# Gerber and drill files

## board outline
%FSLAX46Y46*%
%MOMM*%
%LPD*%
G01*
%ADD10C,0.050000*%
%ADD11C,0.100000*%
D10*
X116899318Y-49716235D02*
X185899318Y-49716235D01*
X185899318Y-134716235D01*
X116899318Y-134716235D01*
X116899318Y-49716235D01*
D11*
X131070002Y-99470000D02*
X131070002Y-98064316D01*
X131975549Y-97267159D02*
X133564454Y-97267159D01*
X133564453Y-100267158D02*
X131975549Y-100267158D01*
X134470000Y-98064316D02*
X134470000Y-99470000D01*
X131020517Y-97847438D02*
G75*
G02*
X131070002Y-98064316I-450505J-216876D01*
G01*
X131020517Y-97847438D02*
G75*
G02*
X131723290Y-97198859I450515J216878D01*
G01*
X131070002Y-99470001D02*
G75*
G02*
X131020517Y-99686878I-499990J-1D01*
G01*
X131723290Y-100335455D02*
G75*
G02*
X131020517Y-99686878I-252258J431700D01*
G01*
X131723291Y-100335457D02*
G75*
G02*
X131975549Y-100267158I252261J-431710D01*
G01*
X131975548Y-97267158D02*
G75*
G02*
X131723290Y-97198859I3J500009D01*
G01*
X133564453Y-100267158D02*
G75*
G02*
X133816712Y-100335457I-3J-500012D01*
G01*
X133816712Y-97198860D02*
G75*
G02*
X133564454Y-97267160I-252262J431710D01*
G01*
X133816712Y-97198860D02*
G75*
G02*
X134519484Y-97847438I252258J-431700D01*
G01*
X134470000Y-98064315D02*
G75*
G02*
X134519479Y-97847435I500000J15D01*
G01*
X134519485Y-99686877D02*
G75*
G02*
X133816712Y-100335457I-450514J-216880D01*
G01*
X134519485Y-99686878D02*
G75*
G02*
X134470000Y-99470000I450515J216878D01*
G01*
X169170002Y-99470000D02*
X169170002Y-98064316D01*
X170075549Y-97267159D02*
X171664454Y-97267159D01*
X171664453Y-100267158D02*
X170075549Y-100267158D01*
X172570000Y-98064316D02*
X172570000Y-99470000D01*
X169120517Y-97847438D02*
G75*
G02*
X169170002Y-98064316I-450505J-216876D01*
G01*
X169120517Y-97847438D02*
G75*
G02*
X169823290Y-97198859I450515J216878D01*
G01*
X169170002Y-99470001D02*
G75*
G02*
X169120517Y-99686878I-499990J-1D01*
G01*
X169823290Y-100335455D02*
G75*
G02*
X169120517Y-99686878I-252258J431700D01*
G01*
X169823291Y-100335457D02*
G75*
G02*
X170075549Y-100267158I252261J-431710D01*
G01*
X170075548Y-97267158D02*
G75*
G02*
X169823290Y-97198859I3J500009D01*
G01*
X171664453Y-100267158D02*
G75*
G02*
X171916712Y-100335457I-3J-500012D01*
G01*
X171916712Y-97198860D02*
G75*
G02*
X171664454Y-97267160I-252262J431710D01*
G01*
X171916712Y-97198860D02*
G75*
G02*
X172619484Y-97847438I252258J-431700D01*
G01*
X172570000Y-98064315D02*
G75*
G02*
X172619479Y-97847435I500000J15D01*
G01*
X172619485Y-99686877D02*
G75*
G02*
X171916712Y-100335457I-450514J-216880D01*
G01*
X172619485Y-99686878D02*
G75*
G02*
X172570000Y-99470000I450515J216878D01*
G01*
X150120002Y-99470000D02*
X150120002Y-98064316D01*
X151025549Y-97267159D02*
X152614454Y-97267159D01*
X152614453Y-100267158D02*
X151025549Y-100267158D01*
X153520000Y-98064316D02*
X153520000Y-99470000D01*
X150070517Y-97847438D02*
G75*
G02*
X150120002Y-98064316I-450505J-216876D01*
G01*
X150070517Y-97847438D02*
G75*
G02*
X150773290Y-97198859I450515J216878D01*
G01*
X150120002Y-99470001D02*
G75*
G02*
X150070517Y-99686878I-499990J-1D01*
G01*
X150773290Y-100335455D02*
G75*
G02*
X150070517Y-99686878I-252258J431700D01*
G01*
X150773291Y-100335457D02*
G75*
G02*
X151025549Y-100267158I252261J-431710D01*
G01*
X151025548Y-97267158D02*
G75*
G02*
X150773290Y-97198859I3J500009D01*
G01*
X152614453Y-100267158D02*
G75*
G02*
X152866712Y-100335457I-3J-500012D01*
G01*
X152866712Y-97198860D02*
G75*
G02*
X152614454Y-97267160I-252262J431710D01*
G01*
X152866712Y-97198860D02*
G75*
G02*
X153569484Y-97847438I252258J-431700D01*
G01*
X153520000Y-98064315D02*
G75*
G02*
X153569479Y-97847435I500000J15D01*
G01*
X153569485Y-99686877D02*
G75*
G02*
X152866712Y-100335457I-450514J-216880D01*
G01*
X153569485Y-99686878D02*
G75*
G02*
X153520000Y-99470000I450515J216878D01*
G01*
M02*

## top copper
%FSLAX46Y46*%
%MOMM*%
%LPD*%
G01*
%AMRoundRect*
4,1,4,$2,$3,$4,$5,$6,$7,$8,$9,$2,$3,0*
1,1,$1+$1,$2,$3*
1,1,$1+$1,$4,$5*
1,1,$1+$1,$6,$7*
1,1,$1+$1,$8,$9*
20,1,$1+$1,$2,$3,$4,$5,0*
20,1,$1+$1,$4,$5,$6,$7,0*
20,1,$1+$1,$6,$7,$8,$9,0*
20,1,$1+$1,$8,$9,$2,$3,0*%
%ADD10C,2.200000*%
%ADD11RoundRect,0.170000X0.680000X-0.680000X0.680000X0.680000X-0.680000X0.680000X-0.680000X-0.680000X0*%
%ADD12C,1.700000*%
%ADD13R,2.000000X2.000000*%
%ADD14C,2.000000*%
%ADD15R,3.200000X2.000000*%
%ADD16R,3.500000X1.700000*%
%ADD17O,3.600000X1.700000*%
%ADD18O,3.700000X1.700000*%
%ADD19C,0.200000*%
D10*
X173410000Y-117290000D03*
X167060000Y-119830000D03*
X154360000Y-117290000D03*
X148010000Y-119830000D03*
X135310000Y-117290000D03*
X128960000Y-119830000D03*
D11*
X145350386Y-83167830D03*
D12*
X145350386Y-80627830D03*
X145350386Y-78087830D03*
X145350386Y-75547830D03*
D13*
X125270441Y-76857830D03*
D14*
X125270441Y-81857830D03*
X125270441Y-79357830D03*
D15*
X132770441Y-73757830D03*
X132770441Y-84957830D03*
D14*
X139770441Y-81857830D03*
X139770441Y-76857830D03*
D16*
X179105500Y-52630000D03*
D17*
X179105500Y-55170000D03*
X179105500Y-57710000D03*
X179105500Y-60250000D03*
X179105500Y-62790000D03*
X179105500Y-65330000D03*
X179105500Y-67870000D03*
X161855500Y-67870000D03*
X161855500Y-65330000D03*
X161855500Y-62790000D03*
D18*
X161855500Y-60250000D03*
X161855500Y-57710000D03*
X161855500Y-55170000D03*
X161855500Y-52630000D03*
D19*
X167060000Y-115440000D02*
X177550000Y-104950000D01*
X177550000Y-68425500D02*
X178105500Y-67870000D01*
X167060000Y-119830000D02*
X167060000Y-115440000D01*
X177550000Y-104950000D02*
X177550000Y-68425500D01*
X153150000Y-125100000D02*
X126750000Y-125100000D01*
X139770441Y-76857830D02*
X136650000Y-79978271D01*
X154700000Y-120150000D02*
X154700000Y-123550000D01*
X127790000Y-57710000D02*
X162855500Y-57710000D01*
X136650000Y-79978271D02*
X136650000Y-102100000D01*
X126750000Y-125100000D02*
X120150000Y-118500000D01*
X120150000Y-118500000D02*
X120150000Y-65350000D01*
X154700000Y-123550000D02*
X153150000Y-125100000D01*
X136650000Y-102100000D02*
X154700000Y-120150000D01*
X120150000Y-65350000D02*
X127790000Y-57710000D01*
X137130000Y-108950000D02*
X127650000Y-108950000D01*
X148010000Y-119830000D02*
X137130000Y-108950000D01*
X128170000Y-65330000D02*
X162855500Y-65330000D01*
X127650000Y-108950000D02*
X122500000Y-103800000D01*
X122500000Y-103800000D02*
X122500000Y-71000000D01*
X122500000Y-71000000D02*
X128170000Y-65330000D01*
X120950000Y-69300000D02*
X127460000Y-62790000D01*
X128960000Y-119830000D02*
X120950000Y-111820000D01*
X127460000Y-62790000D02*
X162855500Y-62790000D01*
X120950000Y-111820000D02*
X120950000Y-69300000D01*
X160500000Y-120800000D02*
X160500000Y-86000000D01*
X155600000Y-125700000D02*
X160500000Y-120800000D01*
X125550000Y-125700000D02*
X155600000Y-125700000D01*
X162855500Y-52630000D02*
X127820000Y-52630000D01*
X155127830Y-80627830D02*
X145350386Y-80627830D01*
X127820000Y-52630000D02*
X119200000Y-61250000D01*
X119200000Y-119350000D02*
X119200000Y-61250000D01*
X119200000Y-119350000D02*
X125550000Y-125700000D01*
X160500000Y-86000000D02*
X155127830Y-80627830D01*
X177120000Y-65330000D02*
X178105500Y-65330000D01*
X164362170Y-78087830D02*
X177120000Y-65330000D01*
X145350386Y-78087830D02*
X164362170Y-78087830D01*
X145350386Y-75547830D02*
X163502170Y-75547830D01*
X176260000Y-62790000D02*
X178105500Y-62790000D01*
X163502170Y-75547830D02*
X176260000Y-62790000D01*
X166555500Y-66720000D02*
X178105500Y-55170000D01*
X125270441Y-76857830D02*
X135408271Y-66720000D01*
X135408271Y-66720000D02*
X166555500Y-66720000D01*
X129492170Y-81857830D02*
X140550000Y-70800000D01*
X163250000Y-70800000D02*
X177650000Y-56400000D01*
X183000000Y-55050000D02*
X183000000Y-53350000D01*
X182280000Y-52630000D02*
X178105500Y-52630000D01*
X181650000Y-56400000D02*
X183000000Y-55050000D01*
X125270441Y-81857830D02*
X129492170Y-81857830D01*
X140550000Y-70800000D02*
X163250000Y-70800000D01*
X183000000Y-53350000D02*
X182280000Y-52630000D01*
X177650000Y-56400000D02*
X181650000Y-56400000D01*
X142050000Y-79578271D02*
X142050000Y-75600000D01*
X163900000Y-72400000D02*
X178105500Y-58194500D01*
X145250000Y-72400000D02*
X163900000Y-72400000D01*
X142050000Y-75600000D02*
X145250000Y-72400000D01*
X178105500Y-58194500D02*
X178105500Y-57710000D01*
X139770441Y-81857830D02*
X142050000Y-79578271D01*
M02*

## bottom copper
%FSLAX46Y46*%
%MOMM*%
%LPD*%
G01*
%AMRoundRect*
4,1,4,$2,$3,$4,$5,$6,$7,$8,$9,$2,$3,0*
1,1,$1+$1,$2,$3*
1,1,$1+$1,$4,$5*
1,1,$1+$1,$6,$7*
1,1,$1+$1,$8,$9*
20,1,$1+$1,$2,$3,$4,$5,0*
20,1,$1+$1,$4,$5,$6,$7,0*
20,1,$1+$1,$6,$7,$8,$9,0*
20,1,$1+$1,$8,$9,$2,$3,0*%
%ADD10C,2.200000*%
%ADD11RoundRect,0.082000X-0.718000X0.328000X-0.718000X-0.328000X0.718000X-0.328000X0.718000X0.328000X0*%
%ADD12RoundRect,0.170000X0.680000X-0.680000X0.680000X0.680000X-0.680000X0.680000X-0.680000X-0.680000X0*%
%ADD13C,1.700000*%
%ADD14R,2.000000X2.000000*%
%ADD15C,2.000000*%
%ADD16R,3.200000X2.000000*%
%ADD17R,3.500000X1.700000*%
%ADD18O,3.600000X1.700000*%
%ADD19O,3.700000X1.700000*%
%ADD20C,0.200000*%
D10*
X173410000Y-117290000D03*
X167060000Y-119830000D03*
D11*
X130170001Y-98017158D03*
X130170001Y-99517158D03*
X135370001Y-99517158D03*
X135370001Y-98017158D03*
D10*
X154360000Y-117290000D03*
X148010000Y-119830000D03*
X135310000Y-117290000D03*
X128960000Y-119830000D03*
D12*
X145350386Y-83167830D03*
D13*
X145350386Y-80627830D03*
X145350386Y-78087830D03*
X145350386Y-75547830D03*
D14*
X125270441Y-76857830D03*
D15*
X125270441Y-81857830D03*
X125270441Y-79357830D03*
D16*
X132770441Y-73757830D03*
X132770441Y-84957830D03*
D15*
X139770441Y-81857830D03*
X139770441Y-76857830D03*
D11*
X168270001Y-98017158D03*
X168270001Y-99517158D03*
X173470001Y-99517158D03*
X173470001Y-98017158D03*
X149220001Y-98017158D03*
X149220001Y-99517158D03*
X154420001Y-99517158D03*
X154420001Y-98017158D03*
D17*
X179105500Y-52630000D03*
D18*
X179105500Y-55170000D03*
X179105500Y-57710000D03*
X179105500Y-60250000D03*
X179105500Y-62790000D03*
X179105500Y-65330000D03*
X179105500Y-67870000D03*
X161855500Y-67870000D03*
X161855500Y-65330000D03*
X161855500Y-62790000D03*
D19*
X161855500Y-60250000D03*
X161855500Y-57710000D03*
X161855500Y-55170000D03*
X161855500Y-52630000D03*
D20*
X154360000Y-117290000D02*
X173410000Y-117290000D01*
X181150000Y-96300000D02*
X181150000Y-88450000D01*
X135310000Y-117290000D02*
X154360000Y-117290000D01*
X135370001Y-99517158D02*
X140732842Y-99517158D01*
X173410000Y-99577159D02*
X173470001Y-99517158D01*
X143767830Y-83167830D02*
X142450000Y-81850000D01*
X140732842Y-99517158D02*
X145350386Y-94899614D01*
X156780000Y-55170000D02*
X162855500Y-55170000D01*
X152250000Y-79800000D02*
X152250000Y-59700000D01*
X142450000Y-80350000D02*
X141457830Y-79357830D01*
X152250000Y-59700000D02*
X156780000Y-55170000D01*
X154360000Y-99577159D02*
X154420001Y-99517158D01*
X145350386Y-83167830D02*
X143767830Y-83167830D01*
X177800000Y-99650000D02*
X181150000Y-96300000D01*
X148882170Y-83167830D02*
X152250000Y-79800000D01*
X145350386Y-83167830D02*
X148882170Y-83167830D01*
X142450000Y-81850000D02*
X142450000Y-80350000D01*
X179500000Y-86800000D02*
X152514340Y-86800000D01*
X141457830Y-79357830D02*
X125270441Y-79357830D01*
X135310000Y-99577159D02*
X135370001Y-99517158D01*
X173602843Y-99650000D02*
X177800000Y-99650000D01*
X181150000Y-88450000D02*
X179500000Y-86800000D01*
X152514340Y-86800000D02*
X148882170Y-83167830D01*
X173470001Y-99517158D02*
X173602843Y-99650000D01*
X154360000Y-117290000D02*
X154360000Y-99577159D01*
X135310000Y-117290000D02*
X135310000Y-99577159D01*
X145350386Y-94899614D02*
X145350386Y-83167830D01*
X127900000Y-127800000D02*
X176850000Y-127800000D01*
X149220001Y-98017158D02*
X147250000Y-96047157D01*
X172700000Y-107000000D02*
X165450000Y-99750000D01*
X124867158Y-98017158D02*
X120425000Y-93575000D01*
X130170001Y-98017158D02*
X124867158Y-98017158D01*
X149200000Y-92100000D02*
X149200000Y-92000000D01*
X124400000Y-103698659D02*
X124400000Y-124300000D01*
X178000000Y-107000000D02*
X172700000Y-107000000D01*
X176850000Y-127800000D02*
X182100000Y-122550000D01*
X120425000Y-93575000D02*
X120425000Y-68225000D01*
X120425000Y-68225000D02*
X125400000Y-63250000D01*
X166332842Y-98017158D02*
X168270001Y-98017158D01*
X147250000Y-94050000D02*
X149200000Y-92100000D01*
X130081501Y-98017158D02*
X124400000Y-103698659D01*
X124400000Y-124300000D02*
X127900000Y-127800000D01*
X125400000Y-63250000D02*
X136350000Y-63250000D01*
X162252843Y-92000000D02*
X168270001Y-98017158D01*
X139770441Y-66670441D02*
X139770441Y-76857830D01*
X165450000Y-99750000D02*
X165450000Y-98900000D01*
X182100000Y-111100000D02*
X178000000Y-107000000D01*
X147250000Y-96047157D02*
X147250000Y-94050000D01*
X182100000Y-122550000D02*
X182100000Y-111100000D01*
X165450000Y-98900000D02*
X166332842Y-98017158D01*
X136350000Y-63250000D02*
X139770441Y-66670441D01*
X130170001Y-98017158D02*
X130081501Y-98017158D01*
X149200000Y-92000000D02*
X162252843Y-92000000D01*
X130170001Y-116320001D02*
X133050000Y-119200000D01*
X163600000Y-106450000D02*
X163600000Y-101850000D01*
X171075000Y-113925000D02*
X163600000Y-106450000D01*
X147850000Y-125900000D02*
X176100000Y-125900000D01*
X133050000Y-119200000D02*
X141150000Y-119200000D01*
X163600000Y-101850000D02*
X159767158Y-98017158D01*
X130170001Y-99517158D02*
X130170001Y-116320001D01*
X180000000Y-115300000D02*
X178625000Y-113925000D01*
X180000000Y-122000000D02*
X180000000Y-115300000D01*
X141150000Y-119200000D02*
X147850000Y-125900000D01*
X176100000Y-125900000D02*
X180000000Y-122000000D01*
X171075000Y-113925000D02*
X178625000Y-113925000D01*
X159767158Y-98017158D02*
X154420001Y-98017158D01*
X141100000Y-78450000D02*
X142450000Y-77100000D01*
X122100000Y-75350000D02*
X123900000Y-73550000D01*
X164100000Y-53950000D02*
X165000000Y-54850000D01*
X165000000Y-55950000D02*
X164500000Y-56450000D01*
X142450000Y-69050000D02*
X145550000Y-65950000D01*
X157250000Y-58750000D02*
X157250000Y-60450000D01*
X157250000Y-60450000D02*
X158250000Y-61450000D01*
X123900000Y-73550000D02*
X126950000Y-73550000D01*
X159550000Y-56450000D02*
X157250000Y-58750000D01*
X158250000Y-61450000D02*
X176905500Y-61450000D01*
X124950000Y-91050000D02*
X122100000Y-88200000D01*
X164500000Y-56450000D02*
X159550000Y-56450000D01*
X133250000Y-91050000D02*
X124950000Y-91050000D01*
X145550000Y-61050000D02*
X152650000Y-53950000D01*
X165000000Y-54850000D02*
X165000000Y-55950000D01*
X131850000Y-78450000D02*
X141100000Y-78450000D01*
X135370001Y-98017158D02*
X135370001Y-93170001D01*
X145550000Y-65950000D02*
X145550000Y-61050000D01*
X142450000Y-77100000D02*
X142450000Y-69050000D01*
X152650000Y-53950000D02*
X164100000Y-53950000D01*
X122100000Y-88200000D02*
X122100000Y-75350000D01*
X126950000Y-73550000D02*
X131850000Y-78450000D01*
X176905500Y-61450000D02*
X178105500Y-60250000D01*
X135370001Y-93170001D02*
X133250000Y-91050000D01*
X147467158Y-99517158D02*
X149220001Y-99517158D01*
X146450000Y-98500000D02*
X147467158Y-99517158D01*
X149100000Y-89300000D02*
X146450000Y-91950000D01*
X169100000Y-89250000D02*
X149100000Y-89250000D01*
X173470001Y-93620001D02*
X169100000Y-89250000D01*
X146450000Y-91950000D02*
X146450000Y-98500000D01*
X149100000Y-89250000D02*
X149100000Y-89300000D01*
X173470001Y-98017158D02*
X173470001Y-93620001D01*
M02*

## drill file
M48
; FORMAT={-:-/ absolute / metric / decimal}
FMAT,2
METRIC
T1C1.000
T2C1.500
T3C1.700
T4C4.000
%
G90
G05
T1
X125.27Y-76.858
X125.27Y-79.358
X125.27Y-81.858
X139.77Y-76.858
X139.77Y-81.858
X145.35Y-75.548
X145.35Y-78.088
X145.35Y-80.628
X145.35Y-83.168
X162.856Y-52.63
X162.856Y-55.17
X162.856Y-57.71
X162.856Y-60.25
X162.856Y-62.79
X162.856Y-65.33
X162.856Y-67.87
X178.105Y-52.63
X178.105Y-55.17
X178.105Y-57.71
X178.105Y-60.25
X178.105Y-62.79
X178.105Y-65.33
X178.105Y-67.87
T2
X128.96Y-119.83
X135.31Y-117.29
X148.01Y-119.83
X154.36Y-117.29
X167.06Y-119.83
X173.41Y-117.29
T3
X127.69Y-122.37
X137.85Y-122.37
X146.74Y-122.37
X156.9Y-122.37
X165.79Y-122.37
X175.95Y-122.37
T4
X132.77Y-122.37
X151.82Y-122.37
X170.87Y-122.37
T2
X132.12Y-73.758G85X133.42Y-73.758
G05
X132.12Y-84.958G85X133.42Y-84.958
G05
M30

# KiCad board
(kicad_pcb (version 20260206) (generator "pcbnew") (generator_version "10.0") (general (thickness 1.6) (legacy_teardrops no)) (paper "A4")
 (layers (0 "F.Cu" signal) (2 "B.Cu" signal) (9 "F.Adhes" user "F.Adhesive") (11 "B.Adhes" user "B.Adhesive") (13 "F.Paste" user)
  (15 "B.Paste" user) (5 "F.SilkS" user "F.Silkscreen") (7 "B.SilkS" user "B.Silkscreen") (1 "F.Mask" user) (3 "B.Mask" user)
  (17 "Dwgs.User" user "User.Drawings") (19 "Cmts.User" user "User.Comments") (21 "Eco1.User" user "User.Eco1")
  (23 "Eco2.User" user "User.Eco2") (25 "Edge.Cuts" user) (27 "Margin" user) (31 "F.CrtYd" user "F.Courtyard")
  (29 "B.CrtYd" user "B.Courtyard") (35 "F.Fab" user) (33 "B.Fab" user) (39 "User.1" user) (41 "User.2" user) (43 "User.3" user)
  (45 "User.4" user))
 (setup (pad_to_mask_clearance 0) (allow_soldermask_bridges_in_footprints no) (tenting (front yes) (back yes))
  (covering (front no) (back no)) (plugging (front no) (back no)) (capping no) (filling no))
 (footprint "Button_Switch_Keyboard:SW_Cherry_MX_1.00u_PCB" (layer "F.Cu") (at 173.41 117.29)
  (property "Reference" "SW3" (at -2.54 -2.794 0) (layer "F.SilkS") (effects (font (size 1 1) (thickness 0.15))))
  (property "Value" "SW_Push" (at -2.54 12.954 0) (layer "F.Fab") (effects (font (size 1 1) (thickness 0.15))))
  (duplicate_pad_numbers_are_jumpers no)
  (pad "" np_thru_hole circle (at -7.62 5.08) (size 1.7 1.7) (drill 1.7) (layers "*.Cu" "*.Mask"))
  (pad "" np_thru_hole circle (at -2.54 5.08) (size 4 4) (drill 4) (layers "*.Cu" "*.Mask"))
  (pad "" np_thru_hole circle (at 2.54 5.08) (size 1.7 1.7) (drill 1.7) (layers "*.Cu" "*.Mask"))
  (pad "1" thru_hole circle (at 0 0) (size 2.2 2.2) (drill 1.5) (layers "*.Cu" "*.Mask") (remove_unused_layers no) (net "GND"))
  (pad "2" thru_hole circle (at -6.35 2.54) (size 2.2 2.2) (drill 1.5) (layers "*.Cu" "*.Mask") (remove_unused_layers no)
   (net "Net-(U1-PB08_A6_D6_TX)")))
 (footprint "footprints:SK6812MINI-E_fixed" (layer "F.Cu") (at 132.77 98.87)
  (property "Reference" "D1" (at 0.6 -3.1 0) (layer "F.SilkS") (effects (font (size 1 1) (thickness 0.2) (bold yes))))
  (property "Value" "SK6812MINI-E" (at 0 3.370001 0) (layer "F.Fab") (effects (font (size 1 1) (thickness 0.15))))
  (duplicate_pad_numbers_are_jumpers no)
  (fp_line (start -1.699998 0.6) (end -1.699998 -0.805684) (stroke (width 0.1) (type solid)) (layer "Edge.Cuts"))
  (fp_line (start -0.794451 -1.602841) (end 0.794454 -1.602841) (stroke (width 0.1) (type solid)) (layer "Edge.Cuts"))
  (fp_line (start 0.794453 1.397158) (end -0.794451 1.397158) (stroke (width 0.1) (type solid)) (layer "Edge.Cuts"))
  (fp_line (start 1.7 -0.805684) (end 1.7 0.6) (stroke (width 0.1) (type solid)) (layer "Edge.Cuts"))
  (fp_arc (start -1.749483 -1.022562) (mid -1.712526 -0.91691) (end -1.699998 -0.805684) (stroke (width 0.1) (type solid))
   (layer "Edge.Cuts"))
  (fp_arc (start -1.749483 -1.022562) (mid -1.63807 -1.606877) (end -1.04671 -1.671141) (stroke (width 0.1) (type solid))
   (layer "Edge.Cuts"))
  (fp_arc (start -1.699998 0.600001) (mid -1.712526 0.711226) (end -1.749483 0.816878) (stroke (width 0.1) (type solid)) (layer "Edge.Cuts"))
  (fp_arc (start -1.04671 1.465455) (mid -1.638069 1.401192) (end -1.749483 0.816878) (stroke (width 0.1) (type solid)) (layer "Edge.Cuts"))
  (fp_arc (start -1.046709 1.465457) (mid -0.925121 1.414535) (end -0.794451 1.397158) (stroke (width 0.1) (type solid)) (layer "Edge.Cuts"))
  (fp_arc (start -0.794452 -1.602842) (mid -0.925122 -1.620219) (end -1.04671 -1.671141) (stroke (width 0.1) (type solid))
   (layer "Edge.Cuts"))
  (fp_arc (start 0.794453 1.397158) (mid 0.925124 1.414535) (end 1.046712 1.465457) (stroke (width 0.1) (type solid)) (layer "Edge.Cuts"))
  (fp_arc (start 1.046712 -1.67114) (mid 0.925124 -1.620218) (end 0.794454 -1.602841) (stroke (width 0.1) (type solid)) (layer "Edge.Cuts"))
  (fp_arc (start 1.046712 -1.67114) (mid 1.638072 -1.606876) (end 1.749485 -1.022562) (stroke (width 0.1) (type solid)) (layer "Edge.Cuts"))
  (fp_arc (start 1.7 -0.805685) (mid 1.712528 -0.91691) (end 1.749485 -1.022562) (stroke (width 0.1) (type solid)) (layer "Edge.Cuts"))
  (fp_arc (start 1.749485 0.816877) (mid 1.638073 1.401193) (end 1.046712 1.465457) (stroke (width 0.1) (type solid)) (layer "Edge.Cuts"))
  (fp_arc (start 1.749485 0.816878) (mid 1.712528 0.711226) (end 1.7 0.6) (stroke (width 0.1) (type solid)) (layer "Edge.Cuts"))
  (pad "1" smd roundrect (at -2.599999 -0.852842 270) (size 0.82 1.6) (layers "B.Cu" "B.Mask" "B.Paste") (roundrect_rratio 0.1)
   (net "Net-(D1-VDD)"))
  (pad "2" smd roundrect (at -2.599999 0.647158 270) (size 0.82 1.6) (layers "B.Cu" "B.Mask" "B.Paste") (roundrect_rratio 0.1)
   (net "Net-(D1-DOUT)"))
  (pad "3" smd roundrect (at 2.600001 0.647158 270) (size 0.82 1.6) (layers "B.Cu" "B.Mask" "B.Paste") (roundrect_rratio 0.1) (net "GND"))
  (pad "4" smd roundrect (at 2.600001 -0.852842 270) (size 0.82 1.6) (layers "B.Cu" "B.Mask" "B.Paste") (roundrect_rratio 0.1)
   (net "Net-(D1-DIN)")))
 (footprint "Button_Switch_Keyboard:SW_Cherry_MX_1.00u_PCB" (layer "F.Cu") (at 154.36 117.29)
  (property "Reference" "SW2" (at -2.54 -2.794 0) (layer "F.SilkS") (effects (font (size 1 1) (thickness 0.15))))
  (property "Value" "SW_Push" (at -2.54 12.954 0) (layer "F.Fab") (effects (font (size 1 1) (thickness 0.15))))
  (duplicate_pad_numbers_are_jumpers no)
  (pad "" np_thru_hole circle (at -7.62 5.08) (size 1.7 1.7) (drill 1.7) (layers "*.Cu" "*.Mask"))
  (pad "" np_thru_hole circle (at -2.54 5.08) (size 4 4) (drill 4) (layers "*.Cu" "*.Mask"))
  (pad "" np_thru_hole circle (at 2.54 5.08) (size 1.7 1.7) (drill 1.7) (layers "*.Cu" "*.Mask"))
  (pad "1" thru_hole circle (at 0 0) (size 2.2 2.2) (drill 1.5) (layers "*.Cu" "*.Mask") (remove_unused_layers no) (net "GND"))
  (pad "2" thru_hole circle (at -6.35 2.54) (size 2.2 2.2) (drill 1.5) (layers "*.Cu" "*.Mask") (remove_unused_layers no)
   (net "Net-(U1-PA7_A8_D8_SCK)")))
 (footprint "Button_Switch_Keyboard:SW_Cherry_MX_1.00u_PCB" (layer "F.Cu") (at 135.31 117.29)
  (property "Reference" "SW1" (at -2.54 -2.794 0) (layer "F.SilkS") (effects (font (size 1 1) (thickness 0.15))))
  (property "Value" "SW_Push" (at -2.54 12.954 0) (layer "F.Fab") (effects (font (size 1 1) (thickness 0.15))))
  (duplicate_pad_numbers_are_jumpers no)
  (pad "" np_thru_hole circle (at -7.62 5.08) (size 1.7 1.7) (drill 1.7) (layers "*.Cu" "*.Mask"))
  (pad "" np_thru_hole circle (at -2.54 5.08) (size 4 4) (drill 4) (layers "*.Cu" "*.Mask"))
  (pad "" np_thru_hole circle (at 2.54 5.08) (size 1.7 1.7) (drill 1.7) (layers "*.Cu" "*.Mask"))
  (pad "1" thru_hole circle (at 0 0) (size 2.2 2.2) (drill 1.5) (layers "*.Cu" "*.Mask") (remove_unused_layers no) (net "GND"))
  (pad "2" thru_hole circle (at -6.35 2.54) (size 2.2 2.2) (drill 1.5) (layers "*.Cu" "*.Mask") (remove_unused_layers no)
   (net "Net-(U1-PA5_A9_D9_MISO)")))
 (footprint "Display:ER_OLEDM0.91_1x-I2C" (layer "F.Cu") (at 145.350386 83.16783 90)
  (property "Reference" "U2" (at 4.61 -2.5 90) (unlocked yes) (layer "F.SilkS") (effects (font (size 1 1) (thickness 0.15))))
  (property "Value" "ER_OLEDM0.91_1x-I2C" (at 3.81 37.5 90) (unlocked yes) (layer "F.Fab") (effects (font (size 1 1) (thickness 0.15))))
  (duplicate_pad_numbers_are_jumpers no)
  (pad "1" thru_hole roundrect (at 0 0 90) (size 1.7 1.7) (drill 1) (layers "*.Cu" "*.Mask") (remove_unused_layers no)
   (roundrect_rratio 0.1) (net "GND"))
  (pad "2" thru_hole circle (at 2.54 0 90) (size 1.7 1.7) (drill 1) (layers "*.Cu" "*.Mask") (remove_unused_layers no) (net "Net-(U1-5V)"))
  (pad "3" thru_hole circle (at 5.08 0 90) (size 1.7 1.7) (drill 1) (layers "*.Cu" "*.Mask") (remove_unused_layers no)
   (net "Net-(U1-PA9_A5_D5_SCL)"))
  (pad "4" thru_hole circle (at 7.62 0 90) (size 1.7 1.7) (drill 1) (layers "*.Cu" "*.Mask") (remove_unused_layers no)
   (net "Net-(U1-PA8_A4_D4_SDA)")))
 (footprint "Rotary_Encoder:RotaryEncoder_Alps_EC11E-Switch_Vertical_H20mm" (layer "F.Cu") (at 125.270441 76.85783)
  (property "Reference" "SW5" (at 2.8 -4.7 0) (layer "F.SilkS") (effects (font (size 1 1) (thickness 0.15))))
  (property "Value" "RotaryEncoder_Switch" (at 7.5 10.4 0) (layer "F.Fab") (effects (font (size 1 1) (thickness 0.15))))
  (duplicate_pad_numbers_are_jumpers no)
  (pad "A" thru_hole rect (at 0 0) (size 2 2) (drill 1) (layers "*.Cu" "*.Mask") (remove_unused_layers no) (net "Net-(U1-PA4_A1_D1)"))
  (pad "B" thru_hole circle (at 0 5) (size 2 2) (drill 1) (layers "*.Cu" "*.Mask") (remove_unused_layers no) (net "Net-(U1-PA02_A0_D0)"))
  (pad "C" thru_hole circle (at 0 2.5) (size 2 2) (drill 1) (layers "*.Cu" "*.Mask") (remove_unused_layers no) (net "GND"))
  (pad "MP" thru_hole rect (at 7.5 -3.1) (size 3.2 2) (drill oval 2.8 1.5) (layers "*.Cu" "*.Mask") (remove_unused_layers no))
  (pad "MP" thru_hole rect (at 7.5 8.1) (size 3.2 2) (drill oval 2.8 1.5) (layers "*.Cu" "*.Mask") (remove_unused_layers no))
  (pad "S1" thru_hole circle (at 14.5 5) (size 2 2) (drill 1) (layers "*.Cu" "*.Mask") (remove_unused_layers no) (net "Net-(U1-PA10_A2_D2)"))
  (pad "S2" thru_hole circle (at 14.5 0) (size 2 2) (drill 1) (layers "*.Cu" "*.Mask") (remove_unused_layers no) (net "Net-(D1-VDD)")))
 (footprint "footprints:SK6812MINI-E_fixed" (layer "F.Cu") (at 170.87 98.87)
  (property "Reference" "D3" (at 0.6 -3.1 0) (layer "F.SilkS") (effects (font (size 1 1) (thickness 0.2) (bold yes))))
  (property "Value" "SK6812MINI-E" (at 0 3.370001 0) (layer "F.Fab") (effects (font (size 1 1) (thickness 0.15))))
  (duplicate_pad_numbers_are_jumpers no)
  (fp_line (start -1.699998 0.6) (end -1.699998 -0.805684) (stroke (width 0.1) (type solid)) (layer "Edge.Cuts"))
  (fp_line (start -0.794451 -1.602841) (end 0.794454 -1.602841) (stroke (width 0.1) (type solid)) (layer "Edge.Cuts"))
  (fp_line (start 0.794453 1.397158) (end -0.794451 1.397158) (stroke (width 0.1) (type solid)) (layer "Edge.Cuts"))
  (fp_line (start 1.7 -0.805684) (end 1.7 0.6) (stroke (width 0.1) (type solid)) (layer "Edge.Cuts"))
  (fp_arc (start -1.749483 -1.022562) (mid -1.712526 -0.91691) (end -1.699998 -0.805684) (stroke (width 0.1) (type solid))
   (layer "Edge.Cuts"))
  (fp_arc (start -1.749483 -1.022562) (mid -1.63807 -1.606877) (end -1.04671 -1.671141) (stroke (width 0.1) (type solid))
   (layer "Edge.Cuts"))
  (fp_arc (start -1.699998 0.600001) (mid -1.712526 0.711226) (end -1.749483 0.816878) (stroke (width 0.1) (type solid)) (layer "Edge.Cuts"))
  (fp_arc (start -1.04671 1.465455) (mid -1.638069 1.401192) (end -1.749483 0.816878) (stroke (width 0.1) (type solid)) (layer "Edge.Cuts"))
  (fp_arc (start -1.046709 1.465457) (mid -0.925121 1.414535) (end -0.794451 1.397158) (stroke (width 0.1) (type solid)) (layer "Edge.Cuts"))
  (fp_arc (start -0.794452 -1.602842) (mid -0.925122 -1.620219) (end -1.04671 -1.671141) (stroke (width 0.1) (type solid))
   (layer "Edge.Cuts"))
  (fp_arc (start 0.794453 1.397158) (mid 0.925124 1.414535) (end 1.046712 1.465457) (stroke (width 0.1) (type solid)) (layer "Edge.Cuts"))
  (fp_arc (start 1.046712 -1.67114) (mid 0.925124 -1.620218) (end 0.794454 -1.602841) (stroke (width 0.1) (type solid)) (layer "Edge.Cuts"))
  (fp_arc (start 1.046712 -1.67114) (mid 1.638072 -1.606876) (end 1.749485 -1.022562) (stroke (width 0.1) (type solid)) (layer "Edge.Cuts"))
  (fp_arc (start 1.7 -0.805685) (mid 1.712528 -0.91691) (end 1.749485 -1.022562) (stroke (width 0.1) (type solid)) (layer "Edge.Cuts"))
  (fp_arc (start 1.749485 0.816877) (mid 1.638073 1.401193) (end 1.046712 1.465457) (stroke (width 0.1) (type solid)) (layer "Edge.Cuts"))
  (fp_arc (start 1.749485 0.816878) (mid 1.712528 0.711226) (end 1.7 0.6) (stroke (width 0.1) (type solid)) (layer "Edge.Cuts"))
  (pad "1" smd roundrect (at -2.599999 -0.852842 270) (size 0.82 1.6) (layers "B.Cu" "B.Mask" "B.Paste") (roundrect_rratio 0.1)
   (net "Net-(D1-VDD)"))
  (pad "2" smd roundrect (at -2.599999 0.647158 270) (size 0.82 1.6) (layers "B.Cu" "B.Mask" "B.Paste") (roundrect_rratio 0.1)
   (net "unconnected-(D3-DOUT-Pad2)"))
  (pad "3" smd roundrect (at 2.600001 0.647158 270) (size 0.82 1.6) (layers "B.Cu" "B.Mask" "B.Paste") (roundrect_rratio 0.1) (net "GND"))
  (pad "4" smd roundrect (at 2.600001 -0.852842 270) (size 0.82 1.6) (layers "B.Cu" "B.Mask" "B.Paste") (roundrect_rratio 0.1)
   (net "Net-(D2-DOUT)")))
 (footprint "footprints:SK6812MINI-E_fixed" (layer "F.Cu") (at 151.82 98.87)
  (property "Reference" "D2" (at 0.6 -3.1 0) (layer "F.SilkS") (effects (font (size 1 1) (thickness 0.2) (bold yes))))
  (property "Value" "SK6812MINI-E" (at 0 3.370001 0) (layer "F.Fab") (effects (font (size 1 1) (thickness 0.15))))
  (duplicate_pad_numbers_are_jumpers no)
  (fp_line (start -1.699998 0.6) (end -1.699998 -0.805684) (stroke (width 0.1) (type solid)) (layer "Edge.Cuts"))
  (fp_line (start -0.794451 -1.602841) (end 0.794454 -1.602841) (stroke (width 0.1) (type solid)) (layer "Edge.Cuts"))
  (fp_line (start 0.794453 1.397158) (end -0.794451 1.397158) (stroke (width 0.1) (type solid)) (layer "Edge.Cuts"))
  (fp_line (start 1.7 -0.805684) (end 1.7 0.6) (stroke (width 0.1) (type solid)) (layer "Edge.Cuts"))
  (fp_arc (start -1.749483 -1.022562) (mid -1.712526 -0.91691) (end -1.699998 -0.805684) (stroke (width 0.1) (type solid))
   (layer "Edge.Cuts"))
  (fp_arc (start -1.749483 -1.022562) (mid -1.63807 -1.606877) (end -1.04671 -1.671141) (stroke (width 0.1) (type solid))
   (layer "Edge.Cuts"))
  (fp_arc (start -1.699998 0.600001) (mid -1.712526 0.711226) (end -1.749483 0.816878) (stroke (width 0.1) (type solid)) (layer "Edge.Cuts"))
  (fp_arc (start -1.04671 1.465455) (mid -1.638069 1.401192) (end -1.749483 0.816878) (stroke (width 0.1) (type solid)) (layer "Edge.Cuts"))
  (fp_arc (start -1.046709 1.465457) (mid -0.925121 1.414535) (end -0.794451 1.397158) (stroke (width 0.1) (type solid)) (layer "Edge.Cuts"))
  (fp_arc (start -0.794452 -1.602842) (mid -0.925122 -1.620219) (end -1.04671 -1.671141) (stroke (width 0.1) (type solid))
   (layer "Edge.Cuts"))
  (fp_arc (start 0.794453 1.397158) (mid 0.925124 1.414535) (end 1.046712 1.465457) (stroke (width 0.1) (type solid)) (layer "Edge.Cuts"))
  (fp_arc (start 1.046712 -1.67114) (mid 0.925124 -1.620218) (end 0.794454 -1.602841) (stroke (width 0.1) (type solid)) (layer "Edge.Cuts"))
  (fp_arc (start 1.046712 -1.67114) (mid 1.638072 -1.606876) (end 1.749485 -1.022562) (stroke (width 0.1) (type solid)) (layer "Edge.Cuts"))
  (fp_arc (start 1.7 -0.805685) (mid 1.712528 -0.91691) (end 1.749485 -1.022562) (stroke (width 0.1) (type solid)) (layer "Edge.Cuts"))
  (fp_arc (start 1.749485 0.816877) (mid 1.638073 1.401193) (end 1.046712 1.465457) (stroke (width 0.1) (type solid)) (layer "Edge.Cuts"))
  (fp_arc (start 1.749485 0.816878) (mid 1.712528 0.711226) (end 1.7 0.6) (stroke (width 0.1) (type solid)) (layer "Edge.Cuts"))
  (pad "1" smd roundrect (at -2.599999 -0.852842 270) (size 0.82 1.6) (layers "B.Cu" "B.Mask" "B.Paste") (roundrect_rratio 0.1)
   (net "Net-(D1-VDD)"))
  (pad "2" smd roundrect (at -2.599999 0.647158 270) (size 0.82 1.6) (layers "B.Cu" "B.Mask" "B.Paste") (roundrect_rratio 0.1)
   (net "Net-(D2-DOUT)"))
  (pad "3" smd roundrect (at 2.600001 0.647158 270) (size 0.82 1.6) (layers "B.Cu" "B.Mask" "B.Paste") (roundrect_rratio 0.1) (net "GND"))
  (pad "4" smd roundrect (at 2.600001 -0.852842 270) (size 0.82 1.6) (layers "B.Cu" "B.Mask" "B.Paste") (roundrect_rratio 0.1)
   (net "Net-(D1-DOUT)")))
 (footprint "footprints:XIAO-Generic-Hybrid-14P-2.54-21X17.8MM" (layer "B.Cu") (at 170.4805 60.25 180)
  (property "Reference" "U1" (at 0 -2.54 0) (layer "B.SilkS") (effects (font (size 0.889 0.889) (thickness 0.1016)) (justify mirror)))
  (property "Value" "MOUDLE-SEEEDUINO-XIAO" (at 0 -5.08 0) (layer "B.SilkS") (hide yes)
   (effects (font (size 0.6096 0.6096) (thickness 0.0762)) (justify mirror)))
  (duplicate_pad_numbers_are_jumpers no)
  (pad "1" thru_hole rect (at -7.625 7.62 180) (size 3.5 1.7) (drill 1 (offset -1 0)) (layers "*.Cu" "*.Mask") (remove_unused_layers no)
   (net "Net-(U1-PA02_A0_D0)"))
  (pad "2" thru_hole oval (at -7.625 5.08 180) (size 3.6 1.7) (drill 1 (offset -1 0)) (layers "*.Cu" "*.Mask") (remove_unused_layers no)
   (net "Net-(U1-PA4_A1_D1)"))
  (pad "3" thru_hole oval (at -7.625 2.54 180) (size 3.6 1.7) (drill 1 (offset -1 0)) (layers "*.Cu" "*.Mask") (remove_unused_layers no)
   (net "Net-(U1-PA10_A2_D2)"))
  (pad "4" thru_hole oval (at -7.625 0 180) (size 3.6 1.7) (drill 1 (offset -1 0)) (layers "*.Cu" "*.Mask") (remove_unused_layers no)
   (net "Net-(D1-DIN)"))
  (pad "5" thru_hole oval (at -7.625 -2.54 180) (size 3.6 1.7) (drill 1 (offset -1 0)) (layers "*.Cu" "*.Mask") (remove_unused_layers no)
   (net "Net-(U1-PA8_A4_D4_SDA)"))
  (pad "6" thru_hole oval (at -7.625 -5.08) (size 3.6 1.7) (drill 1 (offset 1 0)) (layers "*.Cu" "*.Mask") (remove_unused_layers no)
   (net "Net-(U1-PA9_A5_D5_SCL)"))
  (pad "7" thru_hole oval (at -7.625 -7.62 180) (size 3.6 1.7) (drill 1 (offset -1 0)) (layers "*.Cu" "*.Mask") (remove_unused_layers no)
   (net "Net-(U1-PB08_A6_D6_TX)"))
  (pad "8" thru_hole oval (at 7.625 -7.62 180) (size 3.6 1.7) (drill 1 (offset 1 0)) (layers "*.Cu" "*.Mask") (remove_unused_layers no)
   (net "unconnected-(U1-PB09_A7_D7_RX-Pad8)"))
  (pad "9" thru_hole oval (at 7.625 -5.08 180) (size 3.6 1.7) (drill 1 (offset 1 0)) (layers "*.Cu" "*.Mask") (remove_unused_layers no)
   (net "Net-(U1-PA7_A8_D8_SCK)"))
  (pad "10" thru_hole oval (at 7.625 -2.54 180) (size 3.6 1.7) (drill 1 (offset 1 0)) (layers "*.Cu" "*.Mask") (remove_unused_layers no)
   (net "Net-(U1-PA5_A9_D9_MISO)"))
  (pad "11" thru_hole oval (at 7.625 0 180) (size 3.7 1.7) (drill 1 (offset 1 0)) (layers "*.Cu" "*.Mask") (remove_unused_layers no)
   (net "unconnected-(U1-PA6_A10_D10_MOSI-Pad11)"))
  (pad "12" thru_hole oval (at 7.625 2.54 180) (size 3.7 1.7) (drill 1 (offset 1 0)) (layers "*.Cu" "*.Mask") (remove_unused_layers no)
   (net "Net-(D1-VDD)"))
  (pad "13" thru_hole oval (at 7.625 5.08 180) (size 3.7 1.7) (drill 1 (offset 1 0)) (layers "*.Cu" "*.Mask") (remove_unused_layers no)
   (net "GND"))
  (pad "14" thru_hole oval (at 7.625 7.62 180) (size 3.7 1.7) (drill 1 (offset 1 0)) (layers "*.Cu" "*.Mask") (remove_unused_layers no)
   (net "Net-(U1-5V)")))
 (gr_rect (start 116.899318 49.716235) (end 185.899318 134.716235) (stroke (width 0.05) (type default)) (fill no) (layer "Edge.Cuts"))
 (segment (start 154.36 117.29) (end 173.41 117.29) (width 0.2) (layer "B.Cu") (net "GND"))
 (segment (start 181.15 96.3) (end 181.15 88.45) (width 0.2) (layer "B.Cu") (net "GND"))
 (segment (start 135.31 117.29) (end 154.36 117.29) (width 0.2) (layer "B.Cu") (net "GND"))
 (segment (start 135.370001 99.517158) (end 140.732842 99.517158) (width 0.2) (layer "B.Cu") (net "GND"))
 (segment (start 173.41 99.577159) (end 173.470001 99.517158) (width 0.2) (layer "B.Cu") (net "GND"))
 (segment (start 143.76783 83.16783) (end 142.45 81.85) (width 0.2) (layer "B.Cu") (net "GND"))
 (segment (start 140.732842 99.517158) (end 145.350386 94.899614) (width 0.2) (layer "B.Cu") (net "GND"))
 (segment (start 156.78 55.17) (end 162.8555 55.17) (width 0.2) (layer "B.Cu") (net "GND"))
 (segment (start 152.25 79.8) (end 152.25 59.7) (width 0.2) (layer "B.Cu") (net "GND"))
 (segment (start 142.45 80.35) (end 141.45783 79.35783) (width 0.2) (layer "B.Cu") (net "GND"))
 (segment (start 152.25 59.7) (end 156.78 55.17) (width 0.2) (layer "B.Cu") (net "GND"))
 (segment (start 154.36 99.577159) (end 154.420001 99.517158) (width 0.2) (layer "B.Cu") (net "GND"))
 (segment (start 145.350386 83.16783) (end 143.76783 83.16783) (width 0.2) (layer "B.Cu") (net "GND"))
 (segment (start 177.8 99.65) (end 181.15 96.3) (width 0.2) (layer "B.Cu") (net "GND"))
 (segment (start 148.88217 83.16783) (end 152.25 79.8) (width 0.2) (layer "B.Cu") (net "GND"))
 (segment (start 145.350386 83.16783) (end 148.88217 83.16783) (width 0.2) (layer "B.Cu") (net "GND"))
 (segment (start 142.45 81.85) (end 142.45 80.35) (width 0.2) (layer "B.Cu") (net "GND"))
 (segment (start 179.5 86.8) (end 152.51434 86.8) (width 0.2) (layer "B.Cu") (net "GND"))
 (segment (start 141.45783 79.35783) (end 125.270441 79.35783) (width 0.2) (layer "B.Cu") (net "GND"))
 (segment (start 135.31 99.577159) (end 135.370001 99.517158) (width 0.2) (layer "B.Cu") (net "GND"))
 (segment (start 173.602843 99.65) (end 177.8 99.65) (width 0.2) (layer "B.Cu") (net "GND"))
 (segment (start 181.15 88.45) (end 179.5 86.8) (width 0.2) (layer "B.Cu") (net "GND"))
 (segment (start 152.51434 86.8) (end 148.88217 83.16783) (width 0.2) (layer "B.Cu") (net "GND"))
 (segment (start 173.470001 99.517158) (end 173.602843 99.65) (width 0.2) (layer "B.Cu") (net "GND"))
 (segment (start 154.36 117.29) (end 154.36 99.577159) (width 0.2) (layer "B.Cu") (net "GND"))
 (segment (start 135.31 117.29) (end 135.31 99.577159) (width 0.2) (layer "B.Cu") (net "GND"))
 (segment (start 145.350386 94.899614) (end 145.350386 83.16783) (width 0.2) (layer "B.Cu") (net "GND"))
 (segment (start 167.06 115.44) (end 177.55 104.95) (width 0.2) (layer "F.Cu") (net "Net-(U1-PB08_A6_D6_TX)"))
 (segment (start 177.55 68.4255) (end 178.1055 67.87) (width 0.2) (layer "F.Cu") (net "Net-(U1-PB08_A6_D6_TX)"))
 (segment (start 167.06 119.83) (end 167.06 115.44) (width 0.2) (layer "F.Cu") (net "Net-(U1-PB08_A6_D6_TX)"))
 (segment (start 177.55 104.95) (end 177.55 68.4255) (width 0.2) (layer "F.Cu") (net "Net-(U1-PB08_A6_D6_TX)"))
 (segment (start 153.15 125.1) (end 126.75 125.1) (width 0.2) (layer "F.Cu") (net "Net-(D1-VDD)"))
 (segment (start 139.770441 76.85783) (end 136.65 79.978271) (width 0.2) (layer "F.Cu") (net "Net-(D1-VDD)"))
 (segment (start 154.7 120.15) (end 154.7 123.55) (width 0.2) (layer "F.Cu") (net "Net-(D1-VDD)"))
 (segment (start 127.79 57.71) (end 162.8555 57.71) (width 0.2) (layer "F.Cu") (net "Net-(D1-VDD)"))
 (segment (start 136.65 79.978271) (end 136.65 102.1) (width 0.2) (layer "F.Cu") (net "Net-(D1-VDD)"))
 (segment (start 126.75 125.1) (end 120.15 118.5) (width 0.2) (layer "F.Cu") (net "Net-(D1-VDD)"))
 (segment (start 120.15 118.5) (end 120.15 65.35) (width 0.2) (layer "F.Cu") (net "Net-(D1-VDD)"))
 (segment (start 154.7 123.55) (end 153.15 125.1) (width 0.2) (layer "F.Cu") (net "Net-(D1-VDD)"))
 (segment (start 136.65 102.1) (end 154.7 120.15) (width 0.2) (layer "F.Cu") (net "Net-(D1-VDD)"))
 (segment (start 120.15 65.35) (end 127.79 57.71) (width 0.2) (layer "F.Cu") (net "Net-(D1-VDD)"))
 (segment (start 127.9 127.8) (end 176.85 127.8) (width 0.2) (layer "B.Cu") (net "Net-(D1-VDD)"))
 (segment (start 149.220001 98.017158) (end 147.25 96.047157) (width 0.2) (layer "B.Cu") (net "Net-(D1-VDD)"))
 (segment (start 172.7 107) (end 165.45 99.75) (width 0.2) (layer "B.Cu") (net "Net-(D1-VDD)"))
 (segment (start 124.867158 98.017158) (end 120.425 93.575) (width 0.2) (layer "B.Cu") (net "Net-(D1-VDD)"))
 (segment (start 130.170001 98.017158) (end 124.867158 98.017158) (width 0.2) (layer "B.Cu") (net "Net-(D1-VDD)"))
 (segment (start 149.2 92.1) (end 149.2 92) (width 0.2) (layer "B.Cu") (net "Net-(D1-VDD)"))
 (segment (start 124.4 103.698659) (end 124.4 124.3) (width 0.2) (layer "B.Cu") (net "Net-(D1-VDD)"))
 (segment (start 178 107) (end 172.7 107) (width 0.2) (layer "B.Cu") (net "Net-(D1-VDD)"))
 (segment (start 176.85 127.8) (end 182.1 122.55) (width 0.2) (layer "B.Cu") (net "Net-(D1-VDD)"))
 (segment (start 120.425 93.575) (end 120.425 68.225) (width 0.2) (layer "B.Cu") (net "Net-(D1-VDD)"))
 (segment (start 120.425 68.225) (end 125.4 63.25) (width 0.2) (layer "B.Cu") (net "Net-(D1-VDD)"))
 (segment (start 166.332842 98.017158) (end 168.270001 98.017158) (width 0.2) (layer "B.Cu") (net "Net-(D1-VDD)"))
 (segment (start 147.25 94.05) (end 149.2 92.1) (width 0.2) (layer "B.Cu") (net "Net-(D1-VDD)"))
 (segment (start 130.081501 98.017158) (end 124.4 103.698659) (width 0.2) (layer "B.Cu") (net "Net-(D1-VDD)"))
 (segment (start 124.4 124.3) (end 127.9 127.8) (width 0.2) (layer "B.Cu") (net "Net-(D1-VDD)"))
 (segment (start 125.4 63.25) (end 136.35 63.25) (width 0.2) (layer "B.Cu") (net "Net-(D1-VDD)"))
 (segment (start 162.252843 92) (end 168.270001 98.017158) (width 0.2) (layer "B.Cu") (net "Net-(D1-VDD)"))
 (segment (start 139.770441 66.670441) (end 139.770441 76.85783) (width 0.2) (layer "B.Cu") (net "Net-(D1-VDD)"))
 (segment (start 165.45 99.75) (end 165.45 98.9) (width 0.2) (layer "B.Cu") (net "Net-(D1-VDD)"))
 (segment (start 182.1 111.1) (end 178 107) (width 0.2) (layer "B.Cu") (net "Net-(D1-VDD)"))
 (segment (start 147.25 96.047157) (end 147.25 94.05) (width 0.2) (layer "B.Cu") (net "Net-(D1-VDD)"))
 (segment (start 182.1 122.55) (end 182.1 111.1) (width 0.2) (layer "B.Cu") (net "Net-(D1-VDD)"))
 (segment (start 165.45 98.9) (end 166.332842 98.017158) (width 0.2) (layer "B.Cu") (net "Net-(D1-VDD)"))
 (segment (start 136.35 63.25) (end 139.770441 66.670441) (width 0.2) (layer "B.Cu") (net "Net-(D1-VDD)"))
 (segment (start 130.170001 98.017158) (end 130.081501 98.017158) (width 0.2) (layer "B.Cu") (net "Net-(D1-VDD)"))
 (segment (start 149.2 92) (end 162.252843 92) (width 0.2) (layer "B.Cu") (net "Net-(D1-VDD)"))
 (segment (start 130.170001 116.320001) (end 133.05 119.2) (width 0.2) (layer "B.Cu") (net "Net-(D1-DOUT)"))
 (segment (start 163.6 106.45) (end 163.6 101.85) (width 0.2) (layer "B.Cu") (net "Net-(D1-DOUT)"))
 (segment (start 171.075 113.925) (end 163.6 106.45) (width 0.2) (layer "B.Cu") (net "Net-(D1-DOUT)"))
 (segment (start 147.85 125.9) (end 176.1 125.9) (width 0.2) (layer "B.Cu") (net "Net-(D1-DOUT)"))
 (segment (start 133.05 119.2) (end 141.15 119.2) (width 0.2) (layer "B.Cu") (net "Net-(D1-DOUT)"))
 (segment (start 163.6 101.85) (end 159.767158 98.017158) (width 0.2) (layer "B.Cu") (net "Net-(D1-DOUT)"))
 (segment (start 130.170001 99.517158) (end 130.170001 116.320001) (width 0.2) (layer "B.Cu") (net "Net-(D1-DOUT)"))
 (segment (start 180 115.3) (end 178.625 113.925) (width 0.2) (layer "B.Cu") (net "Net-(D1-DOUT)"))
 (segment (start 180 122) (end 180 115.3) (width 0.2) (layer "B.Cu") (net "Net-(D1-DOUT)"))
 (segment (start 141.15 119.2) (end 147.85 125.9) (width 0.2) (layer "B.Cu") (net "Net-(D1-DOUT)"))
 (segment (start 176.1 125.9) (end 180 122) (width 0.2) (layer "B.Cu") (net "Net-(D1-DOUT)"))
 (segment (start 171.075 113.925) (end 178.625 113.925) (width 0.2) (layer "B.Cu") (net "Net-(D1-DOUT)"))
 (segment (start 159.767158 98.017158) (end 154.420001 98.017158) (width 0.2) (layer "B.Cu") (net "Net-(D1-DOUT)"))
 (segment (start 141.1 78.45) (end 142.45 77.1) (width 0.2) (layer "B.Cu") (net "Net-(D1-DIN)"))
 (segment (start 122.1 75.35) (end 123.9 73.55) (width 0.2) (layer "B.Cu") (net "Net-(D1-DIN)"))
 (segment (start 164.1 53.95) (end 165 54.85) (width 0.2) (layer "B.Cu") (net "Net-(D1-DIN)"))
 (segment (start 165 55.95) (end 164.5 56.45) (width 0.2) (layer "B.Cu") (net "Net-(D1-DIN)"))
 (segment (start 142.45 69.05) (end 145.55 65.95) (width 0.2) (layer "B.Cu") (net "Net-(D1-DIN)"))
 (segment (start 157.25 58.75) (end 157.25 60.45) (width 0.2) (layer "B.Cu") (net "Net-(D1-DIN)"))
 (segment (start 157.25 60.45) (end 158.25 61.45) (width 0.2) (layer "B.Cu") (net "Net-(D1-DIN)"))
 (segment (start 123.9 73.55) (end 126.95 73.55) (width 0.2) (layer "B.Cu") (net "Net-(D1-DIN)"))
 (segment (start 159.55 56.45) (end 157.25 58.75) (width 0.2) (layer "B.Cu") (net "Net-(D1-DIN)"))
 (segment (start 158.25 61.45) (end 176.9055 61.45) (width 0.2) (layer "B.Cu") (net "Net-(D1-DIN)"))
 (segment (start 124.95 91.05) (end 122.1 88.2) (width 0.2) (layer "B.Cu") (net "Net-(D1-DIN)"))
 (segment (start 164.5 56.45) (end 159.55 56.45) (width 0.2) (layer "B.Cu") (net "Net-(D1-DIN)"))
 (segment (start 133.25 91.05) (end 124.95 91.05) (width 0.2) (layer "B.Cu") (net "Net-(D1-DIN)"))
 (segment (start 145.55 61.05) (end 152.65 53.95) (width 0.2) (layer "B.Cu") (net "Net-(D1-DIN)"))
 (segment (start 165 54.85) (end 165 55.95) (width 0.2) (layer "B.Cu") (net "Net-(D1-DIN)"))
 (segment (start 131.85 78.45) (end 141.1 78.45) (width 0.2) (layer "B.Cu") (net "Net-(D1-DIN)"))
 (segment (start 135.370001 98.017158) (end 135.370001 93.170001) (width 0.2) (layer "B.Cu") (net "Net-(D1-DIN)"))
 (segment (start 145.55 65.95) (end 145.55 61.05) (width 0.2) (layer "B.Cu") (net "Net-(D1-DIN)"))
 (segment (start 142.45 77.1) (end 142.45 69.05) (width 0.2) (layer "B.Cu") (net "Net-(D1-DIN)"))
 (segment (start 152.65 53.95) (end 164.1 53.95) (width 0.2) (layer "B.Cu") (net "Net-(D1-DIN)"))
 (segment (start 122.1 88.2) (end 122.1 75.35) (width 0.2) (layer "B.Cu") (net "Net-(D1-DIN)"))
 (segment (start 126.95 73.55) (end 131.85 78.45) (width 0.2) (layer "B.Cu") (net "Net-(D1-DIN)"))
 (segment (start 176.9055 61.45) (end 178.1055 60.25) (width 0.2) (layer "B.Cu") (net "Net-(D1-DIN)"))
 (segment (start 135.370001 93.170001) (end 133.25 91.05) (width 0.2) (layer "B.Cu") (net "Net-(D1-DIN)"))
 (segment (start 137.13 108.95) (end 127.65 108.95) (width 0.2) (layer "F.Cu") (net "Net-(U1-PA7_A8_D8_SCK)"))
 (segment (start 148.01 119.83) (end 137.13 108.95) (width 0.2) (layer "F.Cu") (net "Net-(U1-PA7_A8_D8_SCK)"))
 (segment (start 128.17 65.33) (end 162.8555 65.33) (width 0.2) (layer "F.Cu") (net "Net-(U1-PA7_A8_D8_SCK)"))
 (segment (start 127.65 108.95) (end 122.5 103.8) (width 0.2) (layer "F.Cu") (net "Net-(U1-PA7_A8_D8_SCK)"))
 (segment (start 122.5 103.8) (end 122.5 71) (width 0.2) (layer "F.Cu") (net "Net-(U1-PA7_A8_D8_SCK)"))
 (segment (start 122.5 71) (end 128.17 65.33) (width 0.2) (layer "F.Cu") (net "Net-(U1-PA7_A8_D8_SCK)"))
 (segment (start 120.95 69.3) (end 127.46 62.79) (width 0.2) (layer "F.Cu") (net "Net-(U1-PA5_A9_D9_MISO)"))
 (segment (start 128.96 119.83) (end 120.95 111.82) (width 0.2) (layer "F.Cu") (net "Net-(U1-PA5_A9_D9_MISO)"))
 (segment (start 127.46 62.79) (end 162.8555 62.79) (width 0.2) (layer "F.Cu") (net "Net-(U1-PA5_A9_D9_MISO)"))
 (segment (start 120.95 111.82) (end 120.95 69.3) (width 0.2) (layer "F.Cu") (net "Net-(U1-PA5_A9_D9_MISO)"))
 (segment (start 160.5 120.8) (end 160.5 86) (width 0.2) (layer "F.Cu") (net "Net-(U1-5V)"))
 (segment (start 155.6 125.7) (end 160.5 120.8) (width 0.2) (layer "F.Cu") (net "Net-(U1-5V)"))
 (segment (start 125.55 125.7) (end 155.6 125.7) (width 0.2) (layer "F.Cu") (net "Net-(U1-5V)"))
 (segment (start 162.8555 52.63) (end 127.82 52.63) (width 0.2) (layer "F.Cu") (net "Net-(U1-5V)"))
 (segment (start 155.12783 80.62783) (end 145.350386 80.62783) (width 0.2) (layer "F.Cu") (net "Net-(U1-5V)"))
 (segment (start 127.82 52.63) (end 119.2 61.25) (width 0.2) (layer "F.Cu") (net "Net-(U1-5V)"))
 (segment (start 119.2 119.35) (end 119.2 61.25) (width 0.2) (layer "F.Cu") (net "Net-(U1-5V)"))
 (segment (start 119.2 119.35) (end 125.55 125.7) (width 0.2) (layer "F.Cu") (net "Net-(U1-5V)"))
 (segment (start 160.5 86) (end 155.12783 80.62783) (width 0.2) (layer "F.Cu") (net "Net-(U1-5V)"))
 (segment (start 177.12 65.33) (end 178.1055 65.33) (width 0.2) (layer "F.Cu") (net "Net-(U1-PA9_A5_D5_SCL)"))
 (segment (start 164.36217 78.08783) (end 177.12 65.33) (width 0.2) (layer "F.Cu") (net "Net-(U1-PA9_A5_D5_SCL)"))
 (segment (start 145.350386 78.08783) (end 164.36217 78.08783) (width 0.2) (layer "F.Cu") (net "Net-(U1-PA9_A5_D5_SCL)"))
 (segment (start 145.350386 75.54783) (end 163.50217 75.54783) (width 0.2) (layer "F.Cu") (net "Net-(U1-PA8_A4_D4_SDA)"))
 (segment (start 176.26 62.79) (end 178.1055 62.79) (width 0.2) (layer "F.Cu") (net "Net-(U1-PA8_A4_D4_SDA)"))
 (segment (start 163.50217 75.54783) (end 176.26 62.79) (width 0.2) (layer "F.Cu") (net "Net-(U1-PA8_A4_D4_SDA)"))
 (segment (start 166.5555 66.72) (end 178.1055 55.17) (width 0.2) (layer "F.Cu") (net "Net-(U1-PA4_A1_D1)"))
 (segment (start 125.270441 76.85783) (end 135.408271 66.72) (width 0.2) (layer "F.Cu") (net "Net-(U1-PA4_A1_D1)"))
 (segment (start 135.408271 66.72) (end 166.5555 66.72) (width 0.2) (layer "F.Cu") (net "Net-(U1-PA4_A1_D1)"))
 (segment (start 129.49217 81.85783) (end 140.55 70.8) (width 0.2) (layer "F.Cu") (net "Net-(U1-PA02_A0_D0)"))
 (segment (start 163.25 70.8) (end 177.65 56.4) (width 0.2) (layer "F.Cu") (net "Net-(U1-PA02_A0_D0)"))
 (segment (start 183 55.05) (end 183 53.35) (width 0.2) (layer "F.Cu") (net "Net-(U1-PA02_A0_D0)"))
 (segment (start 182.28 52.63) (end 178.1055 52.63) (width 0.2) (layer "F.Cu") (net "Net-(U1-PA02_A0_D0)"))
 (segment (start 181.65 56.4) (end 183 55.05) (width 0.2) (layer "F.Cu") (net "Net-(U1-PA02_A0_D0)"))
 (segment (start 125.270441 81.85783) (end 129.49217 81.85783) (width 0.2) (layer "F.Cu") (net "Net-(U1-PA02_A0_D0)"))
 (segment (start 140.55 70.8) (end 163.25 70.8) (width 0.2) (layer "F.Cu") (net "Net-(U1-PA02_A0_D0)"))
 (segment (start 183 53.35) (end 182.28 52.63) (width 0.2) (layer "F.Cu") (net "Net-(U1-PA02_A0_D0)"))
 (segment (start 177.65 56.4) (end 181.65 56.4) (width 0.2) (layer "F.Cu") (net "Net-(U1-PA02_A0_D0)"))
 (segment (start 142.05 79.578271) (end 142.05 75.6) (width 0.2) (layer "F.Cu") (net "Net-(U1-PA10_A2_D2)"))
 (segment (start 163.9 72.4) (end 178.1055 58.1945) (width 0.2) (layer "F.Cu") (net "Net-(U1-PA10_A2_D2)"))
 (segment (start 145.25 72.4) (end 163.9 72.4) (width 0.2) (layer "F.Cu") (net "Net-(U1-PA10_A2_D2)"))
 (segment (start 142.05 75.6) (end 145.25 72.4) (width 0.2) (layer "F.Cu") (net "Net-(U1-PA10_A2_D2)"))
 (segment (start 178.1055 58.1945) (end 178.1055 57.71) (width 0.2) (layer "F.Cu") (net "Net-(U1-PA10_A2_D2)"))
 (segment (start 139.770441 81.85783) (end 142.05 79.578271) (width 0.2) (layer "F.Cu") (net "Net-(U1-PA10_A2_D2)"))
 (segment (start 147.467158 99.517158) (end 149.220001 99.517158) (width 0.2) (layer "B.Cu") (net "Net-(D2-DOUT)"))
 (segment (start 146.45 98.5) (end 147.467158 99.517158) (width 0.2) (layer "B.Cu") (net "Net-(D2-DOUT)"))
 (segment (start 149.1 89.3) (end 146.45 91.95) (width 0.2) (layer "B.Cu") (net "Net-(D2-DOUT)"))
 (segment (start 169.1 89.25) (end 149.1 89.25) (width 0.2) (layer "B.Cu") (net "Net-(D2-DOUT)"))
 (segment (start 173.470001 93.620001) (end 169.1 89.25) (width 0.2) (layer "B.Cu") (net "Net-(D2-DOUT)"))
 (segment (start 146.45 91.95) (end 146.45 98.5) (width 0.2) (layer "B.Cu") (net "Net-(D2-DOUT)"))
 (segment (start 149.1 89.25) (end 149.1 89.3) (width 0.2) (layer "B.Cu") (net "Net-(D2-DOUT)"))
 (segment (start 173.470001 98.017158) (end 173.470001 93.620001) (width 0.2) (layer "B.Cu") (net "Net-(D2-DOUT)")))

